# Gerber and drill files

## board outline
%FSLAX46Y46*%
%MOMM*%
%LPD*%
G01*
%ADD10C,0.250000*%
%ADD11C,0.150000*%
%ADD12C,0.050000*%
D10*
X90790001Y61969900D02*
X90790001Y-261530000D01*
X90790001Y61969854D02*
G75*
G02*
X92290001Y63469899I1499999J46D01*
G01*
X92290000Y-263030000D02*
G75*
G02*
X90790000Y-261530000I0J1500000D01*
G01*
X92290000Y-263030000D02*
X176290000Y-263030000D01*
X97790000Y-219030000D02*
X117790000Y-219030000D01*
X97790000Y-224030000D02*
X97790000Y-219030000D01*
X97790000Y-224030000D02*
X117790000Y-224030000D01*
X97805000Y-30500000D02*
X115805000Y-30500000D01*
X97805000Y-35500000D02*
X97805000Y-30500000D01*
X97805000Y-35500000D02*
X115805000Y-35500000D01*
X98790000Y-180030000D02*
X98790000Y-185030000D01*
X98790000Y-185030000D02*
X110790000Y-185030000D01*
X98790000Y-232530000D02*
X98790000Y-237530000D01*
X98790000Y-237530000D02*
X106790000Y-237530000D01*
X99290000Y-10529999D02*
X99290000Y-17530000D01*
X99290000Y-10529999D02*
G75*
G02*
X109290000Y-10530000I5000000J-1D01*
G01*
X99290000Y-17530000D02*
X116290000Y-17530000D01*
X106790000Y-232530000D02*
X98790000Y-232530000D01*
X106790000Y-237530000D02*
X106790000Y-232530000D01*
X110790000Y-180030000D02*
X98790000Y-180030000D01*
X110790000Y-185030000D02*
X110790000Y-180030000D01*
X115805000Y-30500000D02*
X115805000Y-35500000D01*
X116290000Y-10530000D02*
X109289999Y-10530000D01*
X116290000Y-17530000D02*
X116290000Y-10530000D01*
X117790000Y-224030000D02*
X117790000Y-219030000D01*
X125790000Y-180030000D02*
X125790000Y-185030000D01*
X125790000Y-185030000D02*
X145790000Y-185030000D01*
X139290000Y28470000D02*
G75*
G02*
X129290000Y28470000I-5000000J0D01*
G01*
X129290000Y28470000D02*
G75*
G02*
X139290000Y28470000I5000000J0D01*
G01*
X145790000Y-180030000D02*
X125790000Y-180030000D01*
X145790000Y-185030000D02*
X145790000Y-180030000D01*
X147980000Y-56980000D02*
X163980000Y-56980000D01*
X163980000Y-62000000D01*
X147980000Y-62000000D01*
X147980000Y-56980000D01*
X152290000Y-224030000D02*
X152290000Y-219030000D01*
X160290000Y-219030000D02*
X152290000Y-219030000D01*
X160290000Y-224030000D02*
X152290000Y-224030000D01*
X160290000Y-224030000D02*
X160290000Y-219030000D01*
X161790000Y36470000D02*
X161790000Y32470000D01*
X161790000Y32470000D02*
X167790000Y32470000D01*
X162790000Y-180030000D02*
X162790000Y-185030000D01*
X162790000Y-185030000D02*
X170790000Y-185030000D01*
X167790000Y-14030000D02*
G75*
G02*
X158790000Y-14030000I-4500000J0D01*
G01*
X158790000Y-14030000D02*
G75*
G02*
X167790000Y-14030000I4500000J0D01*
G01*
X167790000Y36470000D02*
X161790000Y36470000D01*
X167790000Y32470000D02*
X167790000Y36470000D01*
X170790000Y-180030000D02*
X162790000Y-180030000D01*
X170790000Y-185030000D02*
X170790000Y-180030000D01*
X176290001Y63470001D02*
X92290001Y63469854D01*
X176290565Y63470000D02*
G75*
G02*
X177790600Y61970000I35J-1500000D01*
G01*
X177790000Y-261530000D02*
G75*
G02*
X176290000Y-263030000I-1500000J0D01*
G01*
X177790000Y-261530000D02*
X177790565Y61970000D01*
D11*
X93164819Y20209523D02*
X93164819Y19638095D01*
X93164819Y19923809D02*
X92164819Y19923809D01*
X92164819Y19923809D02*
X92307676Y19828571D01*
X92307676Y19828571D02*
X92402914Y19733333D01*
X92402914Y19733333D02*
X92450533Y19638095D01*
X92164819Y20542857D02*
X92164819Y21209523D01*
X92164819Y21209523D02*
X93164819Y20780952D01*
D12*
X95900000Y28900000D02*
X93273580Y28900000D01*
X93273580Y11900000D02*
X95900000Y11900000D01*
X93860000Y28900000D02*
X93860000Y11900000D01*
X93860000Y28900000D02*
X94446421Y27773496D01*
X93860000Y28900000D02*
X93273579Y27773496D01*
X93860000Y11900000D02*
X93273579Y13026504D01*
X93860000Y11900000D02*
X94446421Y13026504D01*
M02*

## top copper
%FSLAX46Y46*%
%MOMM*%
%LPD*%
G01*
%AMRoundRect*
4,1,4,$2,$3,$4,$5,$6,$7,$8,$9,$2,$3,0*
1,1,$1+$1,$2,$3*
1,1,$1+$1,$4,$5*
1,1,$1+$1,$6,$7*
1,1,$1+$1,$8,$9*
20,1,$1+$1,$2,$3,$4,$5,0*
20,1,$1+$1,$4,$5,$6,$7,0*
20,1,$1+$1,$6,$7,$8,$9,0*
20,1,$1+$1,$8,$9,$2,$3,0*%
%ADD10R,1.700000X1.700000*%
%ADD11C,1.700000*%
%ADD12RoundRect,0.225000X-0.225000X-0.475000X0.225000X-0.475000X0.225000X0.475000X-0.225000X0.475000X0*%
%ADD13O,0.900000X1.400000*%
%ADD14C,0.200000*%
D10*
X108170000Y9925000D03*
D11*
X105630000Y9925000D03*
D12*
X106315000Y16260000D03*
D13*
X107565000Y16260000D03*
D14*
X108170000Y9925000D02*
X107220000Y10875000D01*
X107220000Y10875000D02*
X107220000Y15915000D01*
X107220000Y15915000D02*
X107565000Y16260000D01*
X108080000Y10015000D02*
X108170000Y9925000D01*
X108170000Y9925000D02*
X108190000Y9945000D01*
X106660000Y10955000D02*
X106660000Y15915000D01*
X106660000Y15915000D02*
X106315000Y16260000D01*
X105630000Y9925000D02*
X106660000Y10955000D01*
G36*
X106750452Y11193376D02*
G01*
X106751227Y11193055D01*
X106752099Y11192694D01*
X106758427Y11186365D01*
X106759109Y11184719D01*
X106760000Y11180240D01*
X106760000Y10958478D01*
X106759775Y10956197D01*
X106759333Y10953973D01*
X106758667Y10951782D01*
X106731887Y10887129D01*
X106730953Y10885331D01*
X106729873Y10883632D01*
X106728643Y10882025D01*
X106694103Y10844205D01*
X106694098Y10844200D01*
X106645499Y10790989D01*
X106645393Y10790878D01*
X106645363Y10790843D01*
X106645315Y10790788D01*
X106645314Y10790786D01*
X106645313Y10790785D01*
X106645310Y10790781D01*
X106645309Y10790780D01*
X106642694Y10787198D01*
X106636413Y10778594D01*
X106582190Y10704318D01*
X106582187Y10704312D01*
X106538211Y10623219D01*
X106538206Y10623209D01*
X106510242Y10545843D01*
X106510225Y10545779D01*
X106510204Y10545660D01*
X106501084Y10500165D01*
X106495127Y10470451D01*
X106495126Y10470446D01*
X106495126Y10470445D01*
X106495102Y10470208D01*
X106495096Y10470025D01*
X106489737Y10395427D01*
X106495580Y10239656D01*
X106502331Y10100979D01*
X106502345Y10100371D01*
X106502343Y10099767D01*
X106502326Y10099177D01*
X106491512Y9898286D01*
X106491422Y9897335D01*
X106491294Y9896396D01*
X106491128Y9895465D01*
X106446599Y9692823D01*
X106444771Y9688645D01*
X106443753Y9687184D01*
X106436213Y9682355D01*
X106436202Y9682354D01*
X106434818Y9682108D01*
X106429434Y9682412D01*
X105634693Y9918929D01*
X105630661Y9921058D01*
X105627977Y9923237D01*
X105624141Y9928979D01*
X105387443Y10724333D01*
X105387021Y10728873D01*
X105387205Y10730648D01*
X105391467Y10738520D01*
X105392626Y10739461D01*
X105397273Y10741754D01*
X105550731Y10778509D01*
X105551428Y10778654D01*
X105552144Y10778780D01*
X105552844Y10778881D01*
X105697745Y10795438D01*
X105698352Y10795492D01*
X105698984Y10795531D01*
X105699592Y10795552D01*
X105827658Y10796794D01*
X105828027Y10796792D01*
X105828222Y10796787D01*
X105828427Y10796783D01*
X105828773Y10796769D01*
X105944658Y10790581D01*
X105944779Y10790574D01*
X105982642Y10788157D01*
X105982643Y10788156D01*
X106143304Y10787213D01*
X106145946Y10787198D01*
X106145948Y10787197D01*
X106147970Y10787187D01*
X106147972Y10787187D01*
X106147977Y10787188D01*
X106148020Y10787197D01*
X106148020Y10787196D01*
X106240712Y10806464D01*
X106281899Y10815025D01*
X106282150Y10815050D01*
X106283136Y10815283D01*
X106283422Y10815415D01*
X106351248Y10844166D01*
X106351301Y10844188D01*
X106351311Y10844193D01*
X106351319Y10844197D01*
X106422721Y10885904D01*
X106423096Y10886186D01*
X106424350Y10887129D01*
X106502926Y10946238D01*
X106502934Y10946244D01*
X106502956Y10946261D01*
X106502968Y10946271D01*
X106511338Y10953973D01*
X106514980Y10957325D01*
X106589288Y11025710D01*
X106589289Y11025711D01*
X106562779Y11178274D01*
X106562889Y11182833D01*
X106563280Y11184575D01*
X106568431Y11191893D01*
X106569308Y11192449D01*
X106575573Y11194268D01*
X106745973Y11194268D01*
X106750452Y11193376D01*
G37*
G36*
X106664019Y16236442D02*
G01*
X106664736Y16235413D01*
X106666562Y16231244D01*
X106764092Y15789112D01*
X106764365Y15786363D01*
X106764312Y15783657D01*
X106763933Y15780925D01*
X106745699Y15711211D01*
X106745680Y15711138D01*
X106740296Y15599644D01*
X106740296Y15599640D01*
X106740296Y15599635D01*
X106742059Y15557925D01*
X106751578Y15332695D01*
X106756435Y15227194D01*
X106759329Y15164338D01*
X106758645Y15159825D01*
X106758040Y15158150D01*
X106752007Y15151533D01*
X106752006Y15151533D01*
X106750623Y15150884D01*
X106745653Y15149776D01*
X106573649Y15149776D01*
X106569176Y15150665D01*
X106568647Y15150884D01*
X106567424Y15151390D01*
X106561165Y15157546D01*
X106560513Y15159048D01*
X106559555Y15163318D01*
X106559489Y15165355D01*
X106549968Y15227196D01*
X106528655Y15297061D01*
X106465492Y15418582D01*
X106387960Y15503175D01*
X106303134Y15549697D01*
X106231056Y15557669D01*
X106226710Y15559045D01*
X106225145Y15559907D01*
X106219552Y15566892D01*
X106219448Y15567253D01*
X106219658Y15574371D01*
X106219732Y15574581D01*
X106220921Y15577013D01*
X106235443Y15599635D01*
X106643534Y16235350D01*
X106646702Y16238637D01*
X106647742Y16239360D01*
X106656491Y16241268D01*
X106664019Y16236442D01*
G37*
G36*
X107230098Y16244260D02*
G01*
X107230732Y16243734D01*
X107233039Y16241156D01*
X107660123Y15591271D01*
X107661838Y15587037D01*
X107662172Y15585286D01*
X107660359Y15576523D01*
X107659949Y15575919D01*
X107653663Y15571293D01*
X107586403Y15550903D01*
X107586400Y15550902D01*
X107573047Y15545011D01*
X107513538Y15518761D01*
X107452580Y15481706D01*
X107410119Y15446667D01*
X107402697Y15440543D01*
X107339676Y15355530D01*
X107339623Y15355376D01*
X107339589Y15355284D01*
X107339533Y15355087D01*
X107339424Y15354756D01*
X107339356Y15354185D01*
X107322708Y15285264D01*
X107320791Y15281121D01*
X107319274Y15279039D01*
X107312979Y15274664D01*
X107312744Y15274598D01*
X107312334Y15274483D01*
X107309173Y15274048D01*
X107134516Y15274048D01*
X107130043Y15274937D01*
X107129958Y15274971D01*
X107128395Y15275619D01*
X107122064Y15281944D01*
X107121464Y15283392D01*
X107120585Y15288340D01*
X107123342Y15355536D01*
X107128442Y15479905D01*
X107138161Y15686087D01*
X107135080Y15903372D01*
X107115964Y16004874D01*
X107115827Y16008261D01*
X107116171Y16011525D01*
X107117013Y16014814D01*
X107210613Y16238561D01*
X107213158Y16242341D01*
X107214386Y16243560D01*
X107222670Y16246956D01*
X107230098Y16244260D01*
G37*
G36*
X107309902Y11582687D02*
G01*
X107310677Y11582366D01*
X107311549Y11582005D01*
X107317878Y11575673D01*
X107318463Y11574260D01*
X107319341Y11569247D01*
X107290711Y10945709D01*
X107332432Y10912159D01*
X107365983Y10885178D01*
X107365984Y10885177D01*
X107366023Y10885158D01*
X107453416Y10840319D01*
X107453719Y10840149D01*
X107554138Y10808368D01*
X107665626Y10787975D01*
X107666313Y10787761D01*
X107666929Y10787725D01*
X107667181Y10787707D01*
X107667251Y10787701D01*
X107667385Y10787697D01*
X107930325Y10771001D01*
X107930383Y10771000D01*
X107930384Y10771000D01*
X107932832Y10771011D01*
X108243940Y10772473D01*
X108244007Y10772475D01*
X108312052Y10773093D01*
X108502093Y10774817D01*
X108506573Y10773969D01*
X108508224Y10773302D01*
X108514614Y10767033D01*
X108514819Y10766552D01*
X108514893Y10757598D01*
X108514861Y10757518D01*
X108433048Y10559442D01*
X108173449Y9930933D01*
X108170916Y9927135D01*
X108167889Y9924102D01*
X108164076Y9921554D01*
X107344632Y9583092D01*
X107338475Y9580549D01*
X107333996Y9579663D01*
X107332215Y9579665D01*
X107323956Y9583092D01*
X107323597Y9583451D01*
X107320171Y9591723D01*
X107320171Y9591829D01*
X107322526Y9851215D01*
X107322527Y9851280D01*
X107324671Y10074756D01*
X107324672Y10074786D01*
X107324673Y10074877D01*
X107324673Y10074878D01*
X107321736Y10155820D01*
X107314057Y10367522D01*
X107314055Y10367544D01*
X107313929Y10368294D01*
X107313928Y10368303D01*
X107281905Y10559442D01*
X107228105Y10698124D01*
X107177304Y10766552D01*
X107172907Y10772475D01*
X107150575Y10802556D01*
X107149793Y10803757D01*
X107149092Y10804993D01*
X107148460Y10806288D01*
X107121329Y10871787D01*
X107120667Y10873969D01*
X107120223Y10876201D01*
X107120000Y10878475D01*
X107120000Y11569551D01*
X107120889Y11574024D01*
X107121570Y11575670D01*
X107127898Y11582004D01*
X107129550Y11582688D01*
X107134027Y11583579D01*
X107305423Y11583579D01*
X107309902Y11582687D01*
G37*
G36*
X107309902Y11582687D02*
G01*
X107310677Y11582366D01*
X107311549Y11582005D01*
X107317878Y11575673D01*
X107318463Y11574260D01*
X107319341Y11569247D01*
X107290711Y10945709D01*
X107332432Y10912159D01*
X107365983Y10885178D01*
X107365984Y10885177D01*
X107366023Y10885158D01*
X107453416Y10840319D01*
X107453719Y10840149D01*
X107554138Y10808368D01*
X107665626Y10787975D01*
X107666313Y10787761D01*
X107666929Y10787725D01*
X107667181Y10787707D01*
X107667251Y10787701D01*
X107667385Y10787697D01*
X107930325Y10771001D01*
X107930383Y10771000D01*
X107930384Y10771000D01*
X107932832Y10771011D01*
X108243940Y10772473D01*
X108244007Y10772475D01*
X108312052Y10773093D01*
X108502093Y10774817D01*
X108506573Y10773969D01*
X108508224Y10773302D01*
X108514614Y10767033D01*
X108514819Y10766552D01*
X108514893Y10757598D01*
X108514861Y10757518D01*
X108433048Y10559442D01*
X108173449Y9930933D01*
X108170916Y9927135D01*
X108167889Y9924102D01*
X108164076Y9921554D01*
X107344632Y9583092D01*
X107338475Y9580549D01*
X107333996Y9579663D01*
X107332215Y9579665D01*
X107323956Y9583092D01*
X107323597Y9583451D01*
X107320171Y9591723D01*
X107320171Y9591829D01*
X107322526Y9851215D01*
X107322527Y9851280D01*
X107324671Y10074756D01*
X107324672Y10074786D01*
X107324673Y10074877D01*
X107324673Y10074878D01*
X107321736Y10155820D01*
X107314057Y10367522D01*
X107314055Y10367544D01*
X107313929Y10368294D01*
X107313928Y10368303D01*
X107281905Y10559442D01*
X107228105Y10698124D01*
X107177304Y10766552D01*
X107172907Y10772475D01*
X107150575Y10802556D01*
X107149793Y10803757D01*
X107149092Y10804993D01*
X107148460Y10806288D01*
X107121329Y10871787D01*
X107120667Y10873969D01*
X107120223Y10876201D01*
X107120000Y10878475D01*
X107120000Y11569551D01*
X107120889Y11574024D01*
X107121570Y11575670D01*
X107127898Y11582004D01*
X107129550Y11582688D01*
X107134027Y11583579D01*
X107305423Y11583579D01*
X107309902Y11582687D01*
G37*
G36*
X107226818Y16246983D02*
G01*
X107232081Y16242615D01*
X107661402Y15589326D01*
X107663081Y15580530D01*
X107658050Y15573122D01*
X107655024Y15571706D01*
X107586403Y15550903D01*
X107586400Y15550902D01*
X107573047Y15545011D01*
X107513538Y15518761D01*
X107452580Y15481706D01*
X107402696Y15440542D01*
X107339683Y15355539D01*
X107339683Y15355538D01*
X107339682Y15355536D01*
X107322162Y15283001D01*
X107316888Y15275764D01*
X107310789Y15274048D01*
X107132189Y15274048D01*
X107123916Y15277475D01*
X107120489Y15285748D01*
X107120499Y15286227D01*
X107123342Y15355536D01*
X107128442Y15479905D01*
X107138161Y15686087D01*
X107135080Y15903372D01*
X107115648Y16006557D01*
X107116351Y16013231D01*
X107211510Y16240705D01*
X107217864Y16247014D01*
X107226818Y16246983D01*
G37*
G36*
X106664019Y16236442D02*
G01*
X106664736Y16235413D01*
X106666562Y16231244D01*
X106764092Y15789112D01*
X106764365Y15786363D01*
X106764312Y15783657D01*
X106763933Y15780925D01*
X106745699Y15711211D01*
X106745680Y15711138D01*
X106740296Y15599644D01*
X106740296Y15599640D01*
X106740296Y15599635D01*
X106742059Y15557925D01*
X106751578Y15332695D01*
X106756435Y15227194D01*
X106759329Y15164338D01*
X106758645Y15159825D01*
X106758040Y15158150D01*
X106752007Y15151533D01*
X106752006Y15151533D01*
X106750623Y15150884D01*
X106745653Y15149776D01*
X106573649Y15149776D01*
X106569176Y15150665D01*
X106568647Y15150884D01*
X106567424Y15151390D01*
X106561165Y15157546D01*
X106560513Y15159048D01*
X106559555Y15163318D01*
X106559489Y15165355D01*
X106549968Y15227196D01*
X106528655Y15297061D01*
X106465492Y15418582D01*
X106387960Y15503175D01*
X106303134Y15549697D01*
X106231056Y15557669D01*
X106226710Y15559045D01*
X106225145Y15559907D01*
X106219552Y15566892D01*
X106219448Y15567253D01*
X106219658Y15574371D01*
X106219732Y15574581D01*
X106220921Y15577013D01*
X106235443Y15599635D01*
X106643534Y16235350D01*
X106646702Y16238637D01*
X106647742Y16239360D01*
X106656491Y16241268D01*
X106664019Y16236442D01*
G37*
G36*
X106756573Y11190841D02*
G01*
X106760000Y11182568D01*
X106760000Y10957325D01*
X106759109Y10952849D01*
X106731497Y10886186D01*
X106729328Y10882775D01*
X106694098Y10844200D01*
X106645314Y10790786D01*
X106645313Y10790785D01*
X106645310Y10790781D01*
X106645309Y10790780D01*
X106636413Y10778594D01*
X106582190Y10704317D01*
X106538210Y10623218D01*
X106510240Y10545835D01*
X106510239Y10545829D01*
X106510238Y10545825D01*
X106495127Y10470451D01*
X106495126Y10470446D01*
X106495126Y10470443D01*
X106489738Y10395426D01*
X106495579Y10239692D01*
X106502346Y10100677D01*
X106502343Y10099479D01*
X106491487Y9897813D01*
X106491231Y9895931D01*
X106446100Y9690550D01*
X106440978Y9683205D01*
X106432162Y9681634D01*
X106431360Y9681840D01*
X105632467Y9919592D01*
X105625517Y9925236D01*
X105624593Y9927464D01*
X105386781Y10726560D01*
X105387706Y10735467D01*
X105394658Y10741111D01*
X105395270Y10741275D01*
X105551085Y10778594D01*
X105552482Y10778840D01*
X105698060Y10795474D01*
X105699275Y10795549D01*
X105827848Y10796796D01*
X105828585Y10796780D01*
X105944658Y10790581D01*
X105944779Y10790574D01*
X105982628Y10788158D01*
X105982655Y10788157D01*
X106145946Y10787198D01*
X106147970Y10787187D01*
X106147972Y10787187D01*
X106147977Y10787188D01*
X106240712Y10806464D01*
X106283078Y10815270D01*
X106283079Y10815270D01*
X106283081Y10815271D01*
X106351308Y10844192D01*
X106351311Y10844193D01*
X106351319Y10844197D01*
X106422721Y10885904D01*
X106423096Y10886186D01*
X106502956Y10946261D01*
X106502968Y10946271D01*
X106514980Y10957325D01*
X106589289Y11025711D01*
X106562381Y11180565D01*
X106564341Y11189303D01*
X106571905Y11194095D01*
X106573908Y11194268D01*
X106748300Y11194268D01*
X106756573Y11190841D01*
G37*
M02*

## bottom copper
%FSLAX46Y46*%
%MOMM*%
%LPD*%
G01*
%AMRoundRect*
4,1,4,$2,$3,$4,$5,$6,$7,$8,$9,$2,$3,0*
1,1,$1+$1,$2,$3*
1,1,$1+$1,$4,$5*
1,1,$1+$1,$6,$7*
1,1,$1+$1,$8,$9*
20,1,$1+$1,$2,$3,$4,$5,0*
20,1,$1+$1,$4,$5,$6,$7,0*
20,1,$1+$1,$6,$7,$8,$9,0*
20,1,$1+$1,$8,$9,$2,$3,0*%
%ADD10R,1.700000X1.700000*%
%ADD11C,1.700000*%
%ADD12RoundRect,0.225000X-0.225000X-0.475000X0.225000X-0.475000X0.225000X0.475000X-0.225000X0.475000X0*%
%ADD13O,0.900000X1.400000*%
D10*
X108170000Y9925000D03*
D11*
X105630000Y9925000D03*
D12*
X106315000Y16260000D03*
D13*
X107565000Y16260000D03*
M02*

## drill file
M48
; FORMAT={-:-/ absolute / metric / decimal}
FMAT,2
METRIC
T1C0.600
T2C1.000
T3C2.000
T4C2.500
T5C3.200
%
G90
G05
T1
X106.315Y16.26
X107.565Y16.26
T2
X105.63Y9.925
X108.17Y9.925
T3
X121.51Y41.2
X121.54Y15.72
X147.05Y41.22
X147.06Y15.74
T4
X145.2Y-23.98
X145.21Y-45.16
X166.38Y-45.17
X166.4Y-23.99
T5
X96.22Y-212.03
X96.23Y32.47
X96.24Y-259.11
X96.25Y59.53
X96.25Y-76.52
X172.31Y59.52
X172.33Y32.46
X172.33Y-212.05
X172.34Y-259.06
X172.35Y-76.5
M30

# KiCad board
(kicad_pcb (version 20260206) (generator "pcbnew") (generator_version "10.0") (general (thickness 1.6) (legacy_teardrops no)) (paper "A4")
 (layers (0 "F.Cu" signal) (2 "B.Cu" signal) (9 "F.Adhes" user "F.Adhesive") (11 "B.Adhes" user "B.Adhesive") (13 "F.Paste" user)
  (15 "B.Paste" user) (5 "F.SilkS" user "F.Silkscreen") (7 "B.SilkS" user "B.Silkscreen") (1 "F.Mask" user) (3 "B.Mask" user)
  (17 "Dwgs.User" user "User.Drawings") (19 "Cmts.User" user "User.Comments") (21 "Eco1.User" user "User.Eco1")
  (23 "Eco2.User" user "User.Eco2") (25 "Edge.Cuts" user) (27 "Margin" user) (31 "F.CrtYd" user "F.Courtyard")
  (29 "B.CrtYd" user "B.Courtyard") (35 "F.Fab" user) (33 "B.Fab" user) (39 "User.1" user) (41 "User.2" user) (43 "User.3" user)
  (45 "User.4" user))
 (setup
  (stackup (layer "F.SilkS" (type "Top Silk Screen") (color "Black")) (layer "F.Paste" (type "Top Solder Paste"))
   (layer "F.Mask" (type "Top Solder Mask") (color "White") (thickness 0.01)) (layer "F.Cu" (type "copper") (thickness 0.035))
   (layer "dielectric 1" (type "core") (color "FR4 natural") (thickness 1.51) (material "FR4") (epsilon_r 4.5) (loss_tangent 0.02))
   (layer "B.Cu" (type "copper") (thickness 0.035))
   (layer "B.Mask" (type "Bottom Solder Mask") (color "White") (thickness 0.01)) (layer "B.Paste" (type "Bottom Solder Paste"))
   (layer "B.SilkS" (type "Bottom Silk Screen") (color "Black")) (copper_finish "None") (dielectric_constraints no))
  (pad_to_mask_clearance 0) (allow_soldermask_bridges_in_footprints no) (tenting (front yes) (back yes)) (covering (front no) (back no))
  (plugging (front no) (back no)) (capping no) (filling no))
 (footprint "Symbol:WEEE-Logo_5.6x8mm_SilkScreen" (layer "F.Cu") (at 139.726108 -57.742487)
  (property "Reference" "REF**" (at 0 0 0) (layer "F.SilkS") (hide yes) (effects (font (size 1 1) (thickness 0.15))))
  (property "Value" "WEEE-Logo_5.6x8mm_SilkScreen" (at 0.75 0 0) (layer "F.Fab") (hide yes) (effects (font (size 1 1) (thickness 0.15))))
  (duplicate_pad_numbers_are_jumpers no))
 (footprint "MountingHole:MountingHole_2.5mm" (layer "F.Cu") (at 166.4 23.99)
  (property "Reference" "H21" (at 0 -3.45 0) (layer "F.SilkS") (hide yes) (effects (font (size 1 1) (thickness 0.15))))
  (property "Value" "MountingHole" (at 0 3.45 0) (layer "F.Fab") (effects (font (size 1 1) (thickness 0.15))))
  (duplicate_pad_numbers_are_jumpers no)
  (pad "" np_thru_hole circle (at 0 0) (size 2.5 2.5) (drill 2.5) (layers "*.Cu" "*.Mask")))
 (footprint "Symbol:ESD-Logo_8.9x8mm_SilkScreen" (layer "F.Cu") (at 129.333956 -57.700701)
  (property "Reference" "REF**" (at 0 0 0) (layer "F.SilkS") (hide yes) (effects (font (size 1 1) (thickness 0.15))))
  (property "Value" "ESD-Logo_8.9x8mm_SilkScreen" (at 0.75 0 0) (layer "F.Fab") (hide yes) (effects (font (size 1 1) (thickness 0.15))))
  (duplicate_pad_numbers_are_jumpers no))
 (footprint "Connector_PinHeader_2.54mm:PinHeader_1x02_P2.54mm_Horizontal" (layer "F.Cu") (at 108.17 -9.925 -90)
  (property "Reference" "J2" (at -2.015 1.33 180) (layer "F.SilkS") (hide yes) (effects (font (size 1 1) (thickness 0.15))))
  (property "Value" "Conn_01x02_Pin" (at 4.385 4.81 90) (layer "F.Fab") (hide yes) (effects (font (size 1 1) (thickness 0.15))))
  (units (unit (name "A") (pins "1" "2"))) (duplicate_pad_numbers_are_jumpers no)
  (pad "1" thru_hole rect (at 0 0 270) (size 1.7 1.7) (drill 1) (layers "*.Cu" "*.Mask") (remove_unused_layers no) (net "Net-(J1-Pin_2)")
   (teardrops (best_length_ratio 0.5) (max_length 1) (best_width_ratio 1) (max_width 2) (curved_edges yes) (filter_ratio 0.9) (enabled yes)
    (allow_two_segments yes) (prefer_zone_connections yes)))
  (pad "2" thru_hole circle (at 0 2.54 270) (size 1.7 1.7) (drill 1) (layers "*.Cu" "*.Mask") (remove_unused_layers no)
   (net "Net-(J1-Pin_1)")
   (teardrops (best_length_ratio 0.5) (max_length 1) (best_width_ratio 1) (max_width 2) (curved_edges yes) (filter_ratio 0.9) (enabled yes)
    (allow_two_segments yes) (prefer_zone_connections yes))))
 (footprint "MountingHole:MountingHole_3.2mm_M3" (layer "F.Cu") (at 96.25 76.52)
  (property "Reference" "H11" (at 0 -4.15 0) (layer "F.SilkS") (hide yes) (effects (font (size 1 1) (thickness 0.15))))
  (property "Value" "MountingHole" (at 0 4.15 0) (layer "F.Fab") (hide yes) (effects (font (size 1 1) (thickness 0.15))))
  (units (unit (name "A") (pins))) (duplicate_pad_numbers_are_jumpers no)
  (pad "" np_thru_hole circle (at 0 0) (size 3.2 3.2) (drill 3.2) (layers "*.Cu" "*.Mask")))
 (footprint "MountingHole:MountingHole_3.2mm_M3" (layer "F.Cu") (at 172.31 -59.52)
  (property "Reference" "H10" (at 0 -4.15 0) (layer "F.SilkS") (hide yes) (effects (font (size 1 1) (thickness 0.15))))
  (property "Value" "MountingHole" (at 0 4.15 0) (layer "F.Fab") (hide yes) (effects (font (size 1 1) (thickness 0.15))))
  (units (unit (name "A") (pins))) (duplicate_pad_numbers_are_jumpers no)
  (pad "" np_thru_hole circle (at 0 0) (size 3.2 3.2) (drill 3.2) (layers "*.Cu" "*.Mask")))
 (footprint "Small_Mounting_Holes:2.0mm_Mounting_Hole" (layer "F.Cu") (at 121.56 -15.68)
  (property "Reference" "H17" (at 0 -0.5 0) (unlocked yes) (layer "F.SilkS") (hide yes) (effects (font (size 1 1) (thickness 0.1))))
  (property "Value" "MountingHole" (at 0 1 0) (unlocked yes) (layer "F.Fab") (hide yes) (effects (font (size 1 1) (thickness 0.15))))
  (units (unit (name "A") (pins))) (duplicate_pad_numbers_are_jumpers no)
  (pad "" np_thru_hole circle (at -0.02 -0.04) (size 2 2) (drill 2) (layers "*.Cu" "*.Mask")))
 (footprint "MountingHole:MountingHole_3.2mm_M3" (layer "F.Cu") (at 96.24 259.11)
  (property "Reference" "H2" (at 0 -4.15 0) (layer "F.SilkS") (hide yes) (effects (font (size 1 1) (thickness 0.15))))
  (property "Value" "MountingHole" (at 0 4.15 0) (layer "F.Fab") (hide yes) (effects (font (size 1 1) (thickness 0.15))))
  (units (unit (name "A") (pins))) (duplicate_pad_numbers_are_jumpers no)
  (pad "" np_thru_hole circle (at 0 0) (size 3.2 3.2) (drill 3.2) (layers "*.Cu" "*.Mask")))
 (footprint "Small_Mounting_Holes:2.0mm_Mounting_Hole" (layer "F.Cu") (at 147.08 -15.7)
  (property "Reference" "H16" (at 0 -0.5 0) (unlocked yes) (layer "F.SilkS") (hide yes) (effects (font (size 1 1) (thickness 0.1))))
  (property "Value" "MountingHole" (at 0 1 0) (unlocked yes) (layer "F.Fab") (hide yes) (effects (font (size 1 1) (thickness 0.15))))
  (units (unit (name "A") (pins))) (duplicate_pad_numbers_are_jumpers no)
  (pad "" np_thru_hole circle (at -0.02 -0.04) (size 2 2) (drill 2) (layers "*.Cu" "*.Mask")))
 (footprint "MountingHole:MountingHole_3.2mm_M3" (layer "F.Cu") (at 96.23 -32.47)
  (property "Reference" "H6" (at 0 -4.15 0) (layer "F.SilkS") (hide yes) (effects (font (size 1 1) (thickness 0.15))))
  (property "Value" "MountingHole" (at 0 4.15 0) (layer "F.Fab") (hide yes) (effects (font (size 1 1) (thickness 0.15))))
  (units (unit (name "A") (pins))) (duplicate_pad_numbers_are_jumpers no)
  (pad "" np_thru_hole circle (at 0 0) (size 3.2 3.2) (drill 3.2) (layers "*.Cu" "*.Mask")))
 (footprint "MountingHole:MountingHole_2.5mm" (layer "F.Cu") (at 145.21 45.16)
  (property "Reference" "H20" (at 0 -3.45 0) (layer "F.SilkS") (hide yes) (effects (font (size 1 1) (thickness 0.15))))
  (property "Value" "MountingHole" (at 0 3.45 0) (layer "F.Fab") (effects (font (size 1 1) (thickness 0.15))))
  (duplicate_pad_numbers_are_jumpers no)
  (pad "" np_thru_hole circle (at 0 0) (size 2.5 2.5) (drill 2.5) (layers "*.Cu" "*.Mask")))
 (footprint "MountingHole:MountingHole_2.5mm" (layer "F.Cu") (at 145.2 23.98)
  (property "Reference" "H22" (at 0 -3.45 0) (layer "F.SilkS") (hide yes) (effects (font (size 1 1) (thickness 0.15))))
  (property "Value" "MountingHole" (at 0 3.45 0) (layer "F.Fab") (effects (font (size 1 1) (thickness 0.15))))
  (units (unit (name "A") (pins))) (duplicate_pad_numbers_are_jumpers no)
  (pad "" np_thru_hole circle (at 0 0) (size 2.5 2.5) (drill 2.5) (layers "*.Cu" "*.Mask")))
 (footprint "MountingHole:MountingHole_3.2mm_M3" (layer "F.Cu") (at 96.22 212.03)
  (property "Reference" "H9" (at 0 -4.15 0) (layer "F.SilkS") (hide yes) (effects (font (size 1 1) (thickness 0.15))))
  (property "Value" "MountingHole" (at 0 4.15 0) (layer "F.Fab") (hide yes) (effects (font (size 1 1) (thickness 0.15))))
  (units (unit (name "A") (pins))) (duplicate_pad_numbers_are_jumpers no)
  (pad "" np_thru_hole circle (at 0 0) (size 3.2 3.2) (drill 3.2) (layers "*.Cu" "*.Mask")))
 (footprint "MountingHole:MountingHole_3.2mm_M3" (layer "F.Cu") (at 96.25 -59.53)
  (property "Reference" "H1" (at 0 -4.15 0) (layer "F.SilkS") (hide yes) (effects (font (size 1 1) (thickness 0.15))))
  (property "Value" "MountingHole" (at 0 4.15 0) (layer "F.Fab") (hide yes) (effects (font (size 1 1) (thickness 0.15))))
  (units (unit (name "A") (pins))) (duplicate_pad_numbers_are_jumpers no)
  (pad "" np_thru_hole circle (at 0 0) (size 3.2 3.2) (drill 3.2) (layers "*.Cu" "*.Mask")))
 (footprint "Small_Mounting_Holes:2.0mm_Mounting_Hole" (layer "F.Cu") (at 147.07 -41.18)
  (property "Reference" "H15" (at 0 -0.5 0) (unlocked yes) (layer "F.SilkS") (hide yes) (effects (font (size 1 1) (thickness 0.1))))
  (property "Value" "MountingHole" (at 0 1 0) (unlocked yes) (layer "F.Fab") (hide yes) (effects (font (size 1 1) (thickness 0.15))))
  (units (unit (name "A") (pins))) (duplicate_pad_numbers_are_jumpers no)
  (pad "" np_thru_hole circle (at -0.02 -0.04) (size 2 2) (drill 2) (layers "*.Cu" "*.Mask")))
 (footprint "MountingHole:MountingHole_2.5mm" (layer "F.Cu") (at 166.38 45.17)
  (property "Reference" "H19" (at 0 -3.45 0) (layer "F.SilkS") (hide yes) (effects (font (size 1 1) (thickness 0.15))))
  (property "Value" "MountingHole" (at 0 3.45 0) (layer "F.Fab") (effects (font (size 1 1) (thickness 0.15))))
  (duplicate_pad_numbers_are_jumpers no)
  (pad "" np_thru_hole circle (at 0 0) (size 2.5 2.5) (drill 2.5) (layers "*.Cu" "*.Mask")))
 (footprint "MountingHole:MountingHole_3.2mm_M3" (layer "F.Cu") (at 172.33 212.05)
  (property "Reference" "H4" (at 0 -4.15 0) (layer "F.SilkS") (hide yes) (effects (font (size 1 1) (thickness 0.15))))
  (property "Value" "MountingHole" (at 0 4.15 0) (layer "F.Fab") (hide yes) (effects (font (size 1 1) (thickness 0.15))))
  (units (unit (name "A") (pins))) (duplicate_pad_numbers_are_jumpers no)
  (pad "" np_thru_hole circle (at 0 0) (size 3.2 3.2) (drill 3.2) (layers "*.Cu" "*.Mask")))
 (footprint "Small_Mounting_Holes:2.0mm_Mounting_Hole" (layer "F.Cu") (at 121.53 -41.16)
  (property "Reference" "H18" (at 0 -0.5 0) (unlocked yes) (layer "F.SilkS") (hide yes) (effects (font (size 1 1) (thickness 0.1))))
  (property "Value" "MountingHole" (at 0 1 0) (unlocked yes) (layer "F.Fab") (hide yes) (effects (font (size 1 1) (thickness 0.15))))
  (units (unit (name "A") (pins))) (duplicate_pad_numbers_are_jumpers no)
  (pad "" np_thru_hole circle (at -0.02 -0.04) (size 2 2) (drill 2) (layers "*.Cu" "*.Mask")))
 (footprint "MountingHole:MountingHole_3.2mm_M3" (layer "F.Cu") (at 172.33 -32.46)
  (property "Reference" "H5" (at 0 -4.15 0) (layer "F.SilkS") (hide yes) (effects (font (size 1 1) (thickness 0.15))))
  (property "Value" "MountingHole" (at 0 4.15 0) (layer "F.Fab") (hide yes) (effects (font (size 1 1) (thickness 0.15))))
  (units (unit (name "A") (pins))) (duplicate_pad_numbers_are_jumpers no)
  (pad "" np_thru_hole circle (at 0 0) (size 3.2 3.2) (drill 3.2) (layers "*.Cu" "*.Mask")))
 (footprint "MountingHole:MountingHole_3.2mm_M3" (layer "F.Cu") (at 172.35 76.5)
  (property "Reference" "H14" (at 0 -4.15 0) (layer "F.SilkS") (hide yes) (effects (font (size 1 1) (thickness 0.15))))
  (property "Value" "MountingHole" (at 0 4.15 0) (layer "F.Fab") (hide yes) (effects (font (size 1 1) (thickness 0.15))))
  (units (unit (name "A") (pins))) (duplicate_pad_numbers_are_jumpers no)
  (pad "" np_thru_hole circle (at 0 0) (size 3.2 3.2) (drill 3.2) (layers "*.Cu" "*.Mask")))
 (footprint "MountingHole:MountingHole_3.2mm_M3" (layer "F.Cu") (at 172.34 259.06)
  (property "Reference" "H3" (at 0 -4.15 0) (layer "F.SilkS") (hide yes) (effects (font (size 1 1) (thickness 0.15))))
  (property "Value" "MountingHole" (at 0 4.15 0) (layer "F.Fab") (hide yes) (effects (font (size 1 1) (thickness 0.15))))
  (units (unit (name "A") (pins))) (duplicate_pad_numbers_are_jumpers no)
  (pad "" np_thru_hole circle (at 0 0) (size 3.2 3.2) (drill 3.2) (layers "*.Cu" "*.Mask")))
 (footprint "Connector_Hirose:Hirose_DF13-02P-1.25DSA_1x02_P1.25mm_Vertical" (layer "B.Cu") (at 106.315 -16.26)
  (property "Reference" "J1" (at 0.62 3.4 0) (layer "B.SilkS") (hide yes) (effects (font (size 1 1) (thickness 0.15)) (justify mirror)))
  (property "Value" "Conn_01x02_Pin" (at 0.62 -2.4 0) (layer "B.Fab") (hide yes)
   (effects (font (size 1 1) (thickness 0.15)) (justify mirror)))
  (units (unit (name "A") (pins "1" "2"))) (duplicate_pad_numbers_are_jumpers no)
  (pad "1" thru_hole roundrect (at 0 0) (size 0.9 1.4) (drill 0.6) (layers "*.Cu" "*.Mask") (remove_unused_layers no)
   (roundrect_rratio 0.25) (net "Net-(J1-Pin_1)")
   (teardrops (best_length_ratio 0.5) (max_length 1) (best_width_ratio 1) (max_width 2) (curved_edges yes) (filter_ratio 0.9) (enabled yes)
    (allow_two_segments yes) (prefer_zone_connections yes)))
  (pad "2" thru_hole oval (at 1.25 0) (size 0.9 1.4) (drill 0.6) (layers "*.Cu" "*.Mask") (remove_unused_layers no) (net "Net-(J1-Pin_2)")
   (teardrops (best_length_ratio 0.5) (max_length 1) (best_width_ratio 1) (max_width 2) (curved_edges yes) (filter_ratio 0.9) (enabled yes)
    (allow_two_segments yes) (prefer_zone_connections yes))))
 (gr_line (start 90.790001 -61.9699) (end 90.790001 261.53) (stroke (width 0.25) (type solid)) (layer "Edge.Cuts"))
 (gr_arc (start 90.790001 -61.969854) (mid 91.229341 -63.030514) (end 92.290001 -63.469854) (stroke (width 0.25) (type default))
  (layer "Edge.Cuts"))
 (gr_arc (start 92.29 263.03) (mid 91.22934 262.59066) (end 90.79 261.53) (stroke (width 0.25) (type default)) (layer "Edge.Cuts"))
 (gr_line (start 92.29 263.03) (end 176.29 263.03) (stroke (width 0.25) (type solid)) (layer "Edge.Cuts"))
 (gr_line (start 97.79 219.03) (end 117.79 219.03) (stroke (width 0.25) (type solid)) (layer "Edge.Cuts"))
 (gr_line (start 97.79 224.03) (end 97.79 219.03) (stroke (width 0.25) (type default)) (layer "Edge.Cuts"))
 (gr_line (start 97.79 224.03) (end 117.79 224.03) (stroke (width 0.25) (type default)) (layer "Edge.Cuts"))
 (gr_line (start 97.805 30.5) (end 115.805 30.5) (stroke (width 0.25) (type solid)) (layer "Edge.Cuts"))
 (gr_line (start 97.805 35.5) (end 97.805 30.5) (stroke (width 0.25) (type solid)) (layer "Edge.Cuts"))
 (gr_line (start 97.805 35.5) (end 115.805 35.5) (stroke (width 0.25) (type solid)) (layer "Edge.Cuts"))
 (gr_line (start 98.79 180.03) (end 98.79 185.03) (stroke (width 0.25) (type default)) (layer "Edge.Cuts"))
 (gr_line (start 98.79 185.03) (end 110.79 185.03) (stroke (width 0.25) (type default)) (layer "Edge.Cuts"))
 (gr_line (start 98.79 232.53) (end 98.79 237.53) (stroke (width 0.25) (type default)) (layer "Edge.Cuts"))
 (gr_line (start 98.79 237.53) (end 106.79 237.53) (stroke (width 0.25) (type default)) (layer "Edge.Cuts"))
 (gr_line (start 99.29 10.529999) (end 99.29 17.53) (stroke (width 0.25) (type default)) (layer "Edge.Cuts"))
 (gr_arc (start 99.29 10.529999) (mid 104.29 5.53) (end 109.289999 10.53) (stroke (width 0.25) (type default)) (layer "Edge.Cuts"))
 (gr_line (start 99.29 17.53) (end 116.29 17.53) (stroke (width 0.25) (type default)) (layer "Edge.Cuts"))
 (gr_line (start 106.79 232.53) (end 98.79 232.53) (stroke (width 0.25) (type default)) (layer "Edge.Cuts"))
 (gr_line (start 106.79 237.53) (end 106.79 232.53) (stroke (width 0.25) (type default)) (layer "Edge.Cuts"))
 (gr_line (start 110.79 180.03) (end 98.79 180.03) (stroke (width 0.25) (type default)) (layer "Edge.Cuts"))
 (gr_line (start 110.79 185.03) (end 110.79 180.03) (stroke (width 0.25) (type default)) (layer "Edge.Cuts"))
 (gr_line (start 115.805 30.5) (end 115.805 35.5) (stroke (width 0.25) (type solid)) (layer "Edge.Cuts"))
 (gr_line (start 116.29 10.53) (end 109.289999 10.53) (stroke (width 0.25) (type default)) (layer "Edge.Cuts"))
 (gr_line (start 116.29 17.53) (end 116.29 10.53) (stroke (width 0.25) (type solid)) (layer "Edge.Cuts"))
 (gr_line (start 117.79 224.03) (end 117.79 219.03) (stroke (width 0.25) (type default)) (layer "Edge.Cuts"))
 (gr_line (start 125.79 180.03) (end 125.79 185.03) (stroke (width 0.25) (type default)) (layer "Edge.Cuts"))
 (gr_line (start 125.79 185.03) (end 145.79 185.03) (stroke (width 0.25) (type default)) (layer "Edge.Cuts"))
 (gr_circle (center 134.29 -28.47) (end 139.29 -28.47) (stroke (width 0.25) (type default)) (fill no) (layer "Edge.Cuts"))
 (gr_line (start 145.79 180.03) (end 125.79 180.03) (stroke (width 0.25) (type solid)) (layer "Edge.Cuts"))
 (gr_line (start 145.79 185.03) (end 145.79 180.03) (stroke (width 0.25) (type default)) (layer "Edge.Cuts"))
 (gr_rect (start 147.98 56.98) (end 163.98 62) (stroke (width 0.25) (type solid)) (fill no) (layer "Edge.Cuts"))
 (gr_line (start 152.29 224.03) (end 152.29 219.03) (stroke (width 0.25) (type default)) (layer "Edge.Cuts"))
 (gr_line (start 160.29 219.03) (end 152.29 219.03) (stroke (width 0.25) (type default)) (layer "Edge.Cuts"))
 (gr_line (start 160.29 224.03) (end 152.29 224.03) (stroke (width 0.25) (type default)) (layer "Edge.Cuts"))
 (gr_line (start 160.29 224.03) (end 160.29 219.03) (stroke (width 0.25) (type default)) (layer "Edge.Cuts"))
 (gr_line (start 161.79 -36.47) (end 161.79 -32.47) (stroke (width 0.25) (type default)) (layer "Edge.Cuts"))
 (gr_line (start 161.79 -32.47) (end 167.79 -32.47) (stroke (width 0.25) (type default)) (layer "Edge.Cuts"))
 (gr_line (start 162.79 180.03) (end 162.79 185.03) (stroke (width 0.25) (type default)) (layer "Edge.Cuts"))
 (gr_line (start 162.79 185.03) (end 170.79 185.03) (stroke (width 0.25) (type default)) (layer "Edge.Cuts"))
 (gr_circle (center 163.29 14.03) (end 167.79 14.03) (stroke (width 0.25) (type default)) (fill no) (layer "Edge.Cuts"))
 (gr_line (start 167.79 -36.47) (end 161.79 -36.47) (stroke (width 0.25) (type default)) (layer "Edge.Cuts"))
 (gr_line (start 167.79 -32.47) (end 167.79 -36.47) (stroke (width 0.25) (type default)) (layer "Edge.Cuts"))
 (gr_line (start 170.79 180.03) (end 162.79 180.03) (stroke (width 0.25) (type default)) (layer "Edge.Cuts"))
 (gr_line (start 170.79 185.03) (end 170.79 180.03) (stroke (width 0.25) (type default)) (layer "Edge.Cuts"))
 (gr_line (start 176.290001 -63.470001) (end 92.290001 -63.469854) (stroke (width 0.25) (type solid)) (layer "Edge.Cuts"))
 (gr_arc (start 176.290565 -63.47) (mid 177.351225 -63.03066) (end 177.790565 -61.97) (stroke (width 0.25) (type default))
  (layer "Edge.Cuts"))
 (gr_arc (start 177.79 261.53) (mid 177.35066 262.59066) (end 176.29 263.03) (stroke (width 0.25) (type default)) (layer "Edge.Cuts"))
 (gr_line (start 177.79 261.53) (end 177.790565 -61.97) (stroke (width 0.25) (type solid)) (layer "Edge.Cuts"))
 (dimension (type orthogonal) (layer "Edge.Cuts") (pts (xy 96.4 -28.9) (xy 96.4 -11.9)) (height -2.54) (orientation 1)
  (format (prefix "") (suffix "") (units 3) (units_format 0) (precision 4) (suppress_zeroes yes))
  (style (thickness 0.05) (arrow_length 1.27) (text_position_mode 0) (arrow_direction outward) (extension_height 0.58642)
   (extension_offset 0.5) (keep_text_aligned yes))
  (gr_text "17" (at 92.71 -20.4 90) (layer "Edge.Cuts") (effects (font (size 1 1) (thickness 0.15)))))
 (segment (start 108.17 -9.925) (end 107.22 -10.875) (width 0.2) (layer "F.Cu") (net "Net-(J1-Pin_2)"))
 (segment (start 107.22 -10.875) (end 107.22 -15.915) (width 0.2) (layer "F.Cu") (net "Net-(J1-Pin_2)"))
 (segment (start 107.22 -15.915) (end 107.565 -16.26) (width 0.2) (layer "F.Cu") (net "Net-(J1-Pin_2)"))
 (segment (start 108.08 -10.015) (end 108.17 -9.925) (width 0.2) (layer "F.Cu") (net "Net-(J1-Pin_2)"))
 (segment (start 108.17 -9.925) (end 108.19 -9.945) (width 0.2) (layer "F.Cu") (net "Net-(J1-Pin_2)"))
 (segment (start 106.66 -10.955) (end 106.66 -15.915) (width 0.2) (layer "F.Cu") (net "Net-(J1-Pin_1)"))
 (segment (start 106.66 -15.915) (end 106.315 -16.26) (width 0.2) (layer "F.Cu") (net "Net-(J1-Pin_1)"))
 (segment (start 105.63 -9.925) (end 106.66 -10.955) (width 0.2) (layer "F.Cu") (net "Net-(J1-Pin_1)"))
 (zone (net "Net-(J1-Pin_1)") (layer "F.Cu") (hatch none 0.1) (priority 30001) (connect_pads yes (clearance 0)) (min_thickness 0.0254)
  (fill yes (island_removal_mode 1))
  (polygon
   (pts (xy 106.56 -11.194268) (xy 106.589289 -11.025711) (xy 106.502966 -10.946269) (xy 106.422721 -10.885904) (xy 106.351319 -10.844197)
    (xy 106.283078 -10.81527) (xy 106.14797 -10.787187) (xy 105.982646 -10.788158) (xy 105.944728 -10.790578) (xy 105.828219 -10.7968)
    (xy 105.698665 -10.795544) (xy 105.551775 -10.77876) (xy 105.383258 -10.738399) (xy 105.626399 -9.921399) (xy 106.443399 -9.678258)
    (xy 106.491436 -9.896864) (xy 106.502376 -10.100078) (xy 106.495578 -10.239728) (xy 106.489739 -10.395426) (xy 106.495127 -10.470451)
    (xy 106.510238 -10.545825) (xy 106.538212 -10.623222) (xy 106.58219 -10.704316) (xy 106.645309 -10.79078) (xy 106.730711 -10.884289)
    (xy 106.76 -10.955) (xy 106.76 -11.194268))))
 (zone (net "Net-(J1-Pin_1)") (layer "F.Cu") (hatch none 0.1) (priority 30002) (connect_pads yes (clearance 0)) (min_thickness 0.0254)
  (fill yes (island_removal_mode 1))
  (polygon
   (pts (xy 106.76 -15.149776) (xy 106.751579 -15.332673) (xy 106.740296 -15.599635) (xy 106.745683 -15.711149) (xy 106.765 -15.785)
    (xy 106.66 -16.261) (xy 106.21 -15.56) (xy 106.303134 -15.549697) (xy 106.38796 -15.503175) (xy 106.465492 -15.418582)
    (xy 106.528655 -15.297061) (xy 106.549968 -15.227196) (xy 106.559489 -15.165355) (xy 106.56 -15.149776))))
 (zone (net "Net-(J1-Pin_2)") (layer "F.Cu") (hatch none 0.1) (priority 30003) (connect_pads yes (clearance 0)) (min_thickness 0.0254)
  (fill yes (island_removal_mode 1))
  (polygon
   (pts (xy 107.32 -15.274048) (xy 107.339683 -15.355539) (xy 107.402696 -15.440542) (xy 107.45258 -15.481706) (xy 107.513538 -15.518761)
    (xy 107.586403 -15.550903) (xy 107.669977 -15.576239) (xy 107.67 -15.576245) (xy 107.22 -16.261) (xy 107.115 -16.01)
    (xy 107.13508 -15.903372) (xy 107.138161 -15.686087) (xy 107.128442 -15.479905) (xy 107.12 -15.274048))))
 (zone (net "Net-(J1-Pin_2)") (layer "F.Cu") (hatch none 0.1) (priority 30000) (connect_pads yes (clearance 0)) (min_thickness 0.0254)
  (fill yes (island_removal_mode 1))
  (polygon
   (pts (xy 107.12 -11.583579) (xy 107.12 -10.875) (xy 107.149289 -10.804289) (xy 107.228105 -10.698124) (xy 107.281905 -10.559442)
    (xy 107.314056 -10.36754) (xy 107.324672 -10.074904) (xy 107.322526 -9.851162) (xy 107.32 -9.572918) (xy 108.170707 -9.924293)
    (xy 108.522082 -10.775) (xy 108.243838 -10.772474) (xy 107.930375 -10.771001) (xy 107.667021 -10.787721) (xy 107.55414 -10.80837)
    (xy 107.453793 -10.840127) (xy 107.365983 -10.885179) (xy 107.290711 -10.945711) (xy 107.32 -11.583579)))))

